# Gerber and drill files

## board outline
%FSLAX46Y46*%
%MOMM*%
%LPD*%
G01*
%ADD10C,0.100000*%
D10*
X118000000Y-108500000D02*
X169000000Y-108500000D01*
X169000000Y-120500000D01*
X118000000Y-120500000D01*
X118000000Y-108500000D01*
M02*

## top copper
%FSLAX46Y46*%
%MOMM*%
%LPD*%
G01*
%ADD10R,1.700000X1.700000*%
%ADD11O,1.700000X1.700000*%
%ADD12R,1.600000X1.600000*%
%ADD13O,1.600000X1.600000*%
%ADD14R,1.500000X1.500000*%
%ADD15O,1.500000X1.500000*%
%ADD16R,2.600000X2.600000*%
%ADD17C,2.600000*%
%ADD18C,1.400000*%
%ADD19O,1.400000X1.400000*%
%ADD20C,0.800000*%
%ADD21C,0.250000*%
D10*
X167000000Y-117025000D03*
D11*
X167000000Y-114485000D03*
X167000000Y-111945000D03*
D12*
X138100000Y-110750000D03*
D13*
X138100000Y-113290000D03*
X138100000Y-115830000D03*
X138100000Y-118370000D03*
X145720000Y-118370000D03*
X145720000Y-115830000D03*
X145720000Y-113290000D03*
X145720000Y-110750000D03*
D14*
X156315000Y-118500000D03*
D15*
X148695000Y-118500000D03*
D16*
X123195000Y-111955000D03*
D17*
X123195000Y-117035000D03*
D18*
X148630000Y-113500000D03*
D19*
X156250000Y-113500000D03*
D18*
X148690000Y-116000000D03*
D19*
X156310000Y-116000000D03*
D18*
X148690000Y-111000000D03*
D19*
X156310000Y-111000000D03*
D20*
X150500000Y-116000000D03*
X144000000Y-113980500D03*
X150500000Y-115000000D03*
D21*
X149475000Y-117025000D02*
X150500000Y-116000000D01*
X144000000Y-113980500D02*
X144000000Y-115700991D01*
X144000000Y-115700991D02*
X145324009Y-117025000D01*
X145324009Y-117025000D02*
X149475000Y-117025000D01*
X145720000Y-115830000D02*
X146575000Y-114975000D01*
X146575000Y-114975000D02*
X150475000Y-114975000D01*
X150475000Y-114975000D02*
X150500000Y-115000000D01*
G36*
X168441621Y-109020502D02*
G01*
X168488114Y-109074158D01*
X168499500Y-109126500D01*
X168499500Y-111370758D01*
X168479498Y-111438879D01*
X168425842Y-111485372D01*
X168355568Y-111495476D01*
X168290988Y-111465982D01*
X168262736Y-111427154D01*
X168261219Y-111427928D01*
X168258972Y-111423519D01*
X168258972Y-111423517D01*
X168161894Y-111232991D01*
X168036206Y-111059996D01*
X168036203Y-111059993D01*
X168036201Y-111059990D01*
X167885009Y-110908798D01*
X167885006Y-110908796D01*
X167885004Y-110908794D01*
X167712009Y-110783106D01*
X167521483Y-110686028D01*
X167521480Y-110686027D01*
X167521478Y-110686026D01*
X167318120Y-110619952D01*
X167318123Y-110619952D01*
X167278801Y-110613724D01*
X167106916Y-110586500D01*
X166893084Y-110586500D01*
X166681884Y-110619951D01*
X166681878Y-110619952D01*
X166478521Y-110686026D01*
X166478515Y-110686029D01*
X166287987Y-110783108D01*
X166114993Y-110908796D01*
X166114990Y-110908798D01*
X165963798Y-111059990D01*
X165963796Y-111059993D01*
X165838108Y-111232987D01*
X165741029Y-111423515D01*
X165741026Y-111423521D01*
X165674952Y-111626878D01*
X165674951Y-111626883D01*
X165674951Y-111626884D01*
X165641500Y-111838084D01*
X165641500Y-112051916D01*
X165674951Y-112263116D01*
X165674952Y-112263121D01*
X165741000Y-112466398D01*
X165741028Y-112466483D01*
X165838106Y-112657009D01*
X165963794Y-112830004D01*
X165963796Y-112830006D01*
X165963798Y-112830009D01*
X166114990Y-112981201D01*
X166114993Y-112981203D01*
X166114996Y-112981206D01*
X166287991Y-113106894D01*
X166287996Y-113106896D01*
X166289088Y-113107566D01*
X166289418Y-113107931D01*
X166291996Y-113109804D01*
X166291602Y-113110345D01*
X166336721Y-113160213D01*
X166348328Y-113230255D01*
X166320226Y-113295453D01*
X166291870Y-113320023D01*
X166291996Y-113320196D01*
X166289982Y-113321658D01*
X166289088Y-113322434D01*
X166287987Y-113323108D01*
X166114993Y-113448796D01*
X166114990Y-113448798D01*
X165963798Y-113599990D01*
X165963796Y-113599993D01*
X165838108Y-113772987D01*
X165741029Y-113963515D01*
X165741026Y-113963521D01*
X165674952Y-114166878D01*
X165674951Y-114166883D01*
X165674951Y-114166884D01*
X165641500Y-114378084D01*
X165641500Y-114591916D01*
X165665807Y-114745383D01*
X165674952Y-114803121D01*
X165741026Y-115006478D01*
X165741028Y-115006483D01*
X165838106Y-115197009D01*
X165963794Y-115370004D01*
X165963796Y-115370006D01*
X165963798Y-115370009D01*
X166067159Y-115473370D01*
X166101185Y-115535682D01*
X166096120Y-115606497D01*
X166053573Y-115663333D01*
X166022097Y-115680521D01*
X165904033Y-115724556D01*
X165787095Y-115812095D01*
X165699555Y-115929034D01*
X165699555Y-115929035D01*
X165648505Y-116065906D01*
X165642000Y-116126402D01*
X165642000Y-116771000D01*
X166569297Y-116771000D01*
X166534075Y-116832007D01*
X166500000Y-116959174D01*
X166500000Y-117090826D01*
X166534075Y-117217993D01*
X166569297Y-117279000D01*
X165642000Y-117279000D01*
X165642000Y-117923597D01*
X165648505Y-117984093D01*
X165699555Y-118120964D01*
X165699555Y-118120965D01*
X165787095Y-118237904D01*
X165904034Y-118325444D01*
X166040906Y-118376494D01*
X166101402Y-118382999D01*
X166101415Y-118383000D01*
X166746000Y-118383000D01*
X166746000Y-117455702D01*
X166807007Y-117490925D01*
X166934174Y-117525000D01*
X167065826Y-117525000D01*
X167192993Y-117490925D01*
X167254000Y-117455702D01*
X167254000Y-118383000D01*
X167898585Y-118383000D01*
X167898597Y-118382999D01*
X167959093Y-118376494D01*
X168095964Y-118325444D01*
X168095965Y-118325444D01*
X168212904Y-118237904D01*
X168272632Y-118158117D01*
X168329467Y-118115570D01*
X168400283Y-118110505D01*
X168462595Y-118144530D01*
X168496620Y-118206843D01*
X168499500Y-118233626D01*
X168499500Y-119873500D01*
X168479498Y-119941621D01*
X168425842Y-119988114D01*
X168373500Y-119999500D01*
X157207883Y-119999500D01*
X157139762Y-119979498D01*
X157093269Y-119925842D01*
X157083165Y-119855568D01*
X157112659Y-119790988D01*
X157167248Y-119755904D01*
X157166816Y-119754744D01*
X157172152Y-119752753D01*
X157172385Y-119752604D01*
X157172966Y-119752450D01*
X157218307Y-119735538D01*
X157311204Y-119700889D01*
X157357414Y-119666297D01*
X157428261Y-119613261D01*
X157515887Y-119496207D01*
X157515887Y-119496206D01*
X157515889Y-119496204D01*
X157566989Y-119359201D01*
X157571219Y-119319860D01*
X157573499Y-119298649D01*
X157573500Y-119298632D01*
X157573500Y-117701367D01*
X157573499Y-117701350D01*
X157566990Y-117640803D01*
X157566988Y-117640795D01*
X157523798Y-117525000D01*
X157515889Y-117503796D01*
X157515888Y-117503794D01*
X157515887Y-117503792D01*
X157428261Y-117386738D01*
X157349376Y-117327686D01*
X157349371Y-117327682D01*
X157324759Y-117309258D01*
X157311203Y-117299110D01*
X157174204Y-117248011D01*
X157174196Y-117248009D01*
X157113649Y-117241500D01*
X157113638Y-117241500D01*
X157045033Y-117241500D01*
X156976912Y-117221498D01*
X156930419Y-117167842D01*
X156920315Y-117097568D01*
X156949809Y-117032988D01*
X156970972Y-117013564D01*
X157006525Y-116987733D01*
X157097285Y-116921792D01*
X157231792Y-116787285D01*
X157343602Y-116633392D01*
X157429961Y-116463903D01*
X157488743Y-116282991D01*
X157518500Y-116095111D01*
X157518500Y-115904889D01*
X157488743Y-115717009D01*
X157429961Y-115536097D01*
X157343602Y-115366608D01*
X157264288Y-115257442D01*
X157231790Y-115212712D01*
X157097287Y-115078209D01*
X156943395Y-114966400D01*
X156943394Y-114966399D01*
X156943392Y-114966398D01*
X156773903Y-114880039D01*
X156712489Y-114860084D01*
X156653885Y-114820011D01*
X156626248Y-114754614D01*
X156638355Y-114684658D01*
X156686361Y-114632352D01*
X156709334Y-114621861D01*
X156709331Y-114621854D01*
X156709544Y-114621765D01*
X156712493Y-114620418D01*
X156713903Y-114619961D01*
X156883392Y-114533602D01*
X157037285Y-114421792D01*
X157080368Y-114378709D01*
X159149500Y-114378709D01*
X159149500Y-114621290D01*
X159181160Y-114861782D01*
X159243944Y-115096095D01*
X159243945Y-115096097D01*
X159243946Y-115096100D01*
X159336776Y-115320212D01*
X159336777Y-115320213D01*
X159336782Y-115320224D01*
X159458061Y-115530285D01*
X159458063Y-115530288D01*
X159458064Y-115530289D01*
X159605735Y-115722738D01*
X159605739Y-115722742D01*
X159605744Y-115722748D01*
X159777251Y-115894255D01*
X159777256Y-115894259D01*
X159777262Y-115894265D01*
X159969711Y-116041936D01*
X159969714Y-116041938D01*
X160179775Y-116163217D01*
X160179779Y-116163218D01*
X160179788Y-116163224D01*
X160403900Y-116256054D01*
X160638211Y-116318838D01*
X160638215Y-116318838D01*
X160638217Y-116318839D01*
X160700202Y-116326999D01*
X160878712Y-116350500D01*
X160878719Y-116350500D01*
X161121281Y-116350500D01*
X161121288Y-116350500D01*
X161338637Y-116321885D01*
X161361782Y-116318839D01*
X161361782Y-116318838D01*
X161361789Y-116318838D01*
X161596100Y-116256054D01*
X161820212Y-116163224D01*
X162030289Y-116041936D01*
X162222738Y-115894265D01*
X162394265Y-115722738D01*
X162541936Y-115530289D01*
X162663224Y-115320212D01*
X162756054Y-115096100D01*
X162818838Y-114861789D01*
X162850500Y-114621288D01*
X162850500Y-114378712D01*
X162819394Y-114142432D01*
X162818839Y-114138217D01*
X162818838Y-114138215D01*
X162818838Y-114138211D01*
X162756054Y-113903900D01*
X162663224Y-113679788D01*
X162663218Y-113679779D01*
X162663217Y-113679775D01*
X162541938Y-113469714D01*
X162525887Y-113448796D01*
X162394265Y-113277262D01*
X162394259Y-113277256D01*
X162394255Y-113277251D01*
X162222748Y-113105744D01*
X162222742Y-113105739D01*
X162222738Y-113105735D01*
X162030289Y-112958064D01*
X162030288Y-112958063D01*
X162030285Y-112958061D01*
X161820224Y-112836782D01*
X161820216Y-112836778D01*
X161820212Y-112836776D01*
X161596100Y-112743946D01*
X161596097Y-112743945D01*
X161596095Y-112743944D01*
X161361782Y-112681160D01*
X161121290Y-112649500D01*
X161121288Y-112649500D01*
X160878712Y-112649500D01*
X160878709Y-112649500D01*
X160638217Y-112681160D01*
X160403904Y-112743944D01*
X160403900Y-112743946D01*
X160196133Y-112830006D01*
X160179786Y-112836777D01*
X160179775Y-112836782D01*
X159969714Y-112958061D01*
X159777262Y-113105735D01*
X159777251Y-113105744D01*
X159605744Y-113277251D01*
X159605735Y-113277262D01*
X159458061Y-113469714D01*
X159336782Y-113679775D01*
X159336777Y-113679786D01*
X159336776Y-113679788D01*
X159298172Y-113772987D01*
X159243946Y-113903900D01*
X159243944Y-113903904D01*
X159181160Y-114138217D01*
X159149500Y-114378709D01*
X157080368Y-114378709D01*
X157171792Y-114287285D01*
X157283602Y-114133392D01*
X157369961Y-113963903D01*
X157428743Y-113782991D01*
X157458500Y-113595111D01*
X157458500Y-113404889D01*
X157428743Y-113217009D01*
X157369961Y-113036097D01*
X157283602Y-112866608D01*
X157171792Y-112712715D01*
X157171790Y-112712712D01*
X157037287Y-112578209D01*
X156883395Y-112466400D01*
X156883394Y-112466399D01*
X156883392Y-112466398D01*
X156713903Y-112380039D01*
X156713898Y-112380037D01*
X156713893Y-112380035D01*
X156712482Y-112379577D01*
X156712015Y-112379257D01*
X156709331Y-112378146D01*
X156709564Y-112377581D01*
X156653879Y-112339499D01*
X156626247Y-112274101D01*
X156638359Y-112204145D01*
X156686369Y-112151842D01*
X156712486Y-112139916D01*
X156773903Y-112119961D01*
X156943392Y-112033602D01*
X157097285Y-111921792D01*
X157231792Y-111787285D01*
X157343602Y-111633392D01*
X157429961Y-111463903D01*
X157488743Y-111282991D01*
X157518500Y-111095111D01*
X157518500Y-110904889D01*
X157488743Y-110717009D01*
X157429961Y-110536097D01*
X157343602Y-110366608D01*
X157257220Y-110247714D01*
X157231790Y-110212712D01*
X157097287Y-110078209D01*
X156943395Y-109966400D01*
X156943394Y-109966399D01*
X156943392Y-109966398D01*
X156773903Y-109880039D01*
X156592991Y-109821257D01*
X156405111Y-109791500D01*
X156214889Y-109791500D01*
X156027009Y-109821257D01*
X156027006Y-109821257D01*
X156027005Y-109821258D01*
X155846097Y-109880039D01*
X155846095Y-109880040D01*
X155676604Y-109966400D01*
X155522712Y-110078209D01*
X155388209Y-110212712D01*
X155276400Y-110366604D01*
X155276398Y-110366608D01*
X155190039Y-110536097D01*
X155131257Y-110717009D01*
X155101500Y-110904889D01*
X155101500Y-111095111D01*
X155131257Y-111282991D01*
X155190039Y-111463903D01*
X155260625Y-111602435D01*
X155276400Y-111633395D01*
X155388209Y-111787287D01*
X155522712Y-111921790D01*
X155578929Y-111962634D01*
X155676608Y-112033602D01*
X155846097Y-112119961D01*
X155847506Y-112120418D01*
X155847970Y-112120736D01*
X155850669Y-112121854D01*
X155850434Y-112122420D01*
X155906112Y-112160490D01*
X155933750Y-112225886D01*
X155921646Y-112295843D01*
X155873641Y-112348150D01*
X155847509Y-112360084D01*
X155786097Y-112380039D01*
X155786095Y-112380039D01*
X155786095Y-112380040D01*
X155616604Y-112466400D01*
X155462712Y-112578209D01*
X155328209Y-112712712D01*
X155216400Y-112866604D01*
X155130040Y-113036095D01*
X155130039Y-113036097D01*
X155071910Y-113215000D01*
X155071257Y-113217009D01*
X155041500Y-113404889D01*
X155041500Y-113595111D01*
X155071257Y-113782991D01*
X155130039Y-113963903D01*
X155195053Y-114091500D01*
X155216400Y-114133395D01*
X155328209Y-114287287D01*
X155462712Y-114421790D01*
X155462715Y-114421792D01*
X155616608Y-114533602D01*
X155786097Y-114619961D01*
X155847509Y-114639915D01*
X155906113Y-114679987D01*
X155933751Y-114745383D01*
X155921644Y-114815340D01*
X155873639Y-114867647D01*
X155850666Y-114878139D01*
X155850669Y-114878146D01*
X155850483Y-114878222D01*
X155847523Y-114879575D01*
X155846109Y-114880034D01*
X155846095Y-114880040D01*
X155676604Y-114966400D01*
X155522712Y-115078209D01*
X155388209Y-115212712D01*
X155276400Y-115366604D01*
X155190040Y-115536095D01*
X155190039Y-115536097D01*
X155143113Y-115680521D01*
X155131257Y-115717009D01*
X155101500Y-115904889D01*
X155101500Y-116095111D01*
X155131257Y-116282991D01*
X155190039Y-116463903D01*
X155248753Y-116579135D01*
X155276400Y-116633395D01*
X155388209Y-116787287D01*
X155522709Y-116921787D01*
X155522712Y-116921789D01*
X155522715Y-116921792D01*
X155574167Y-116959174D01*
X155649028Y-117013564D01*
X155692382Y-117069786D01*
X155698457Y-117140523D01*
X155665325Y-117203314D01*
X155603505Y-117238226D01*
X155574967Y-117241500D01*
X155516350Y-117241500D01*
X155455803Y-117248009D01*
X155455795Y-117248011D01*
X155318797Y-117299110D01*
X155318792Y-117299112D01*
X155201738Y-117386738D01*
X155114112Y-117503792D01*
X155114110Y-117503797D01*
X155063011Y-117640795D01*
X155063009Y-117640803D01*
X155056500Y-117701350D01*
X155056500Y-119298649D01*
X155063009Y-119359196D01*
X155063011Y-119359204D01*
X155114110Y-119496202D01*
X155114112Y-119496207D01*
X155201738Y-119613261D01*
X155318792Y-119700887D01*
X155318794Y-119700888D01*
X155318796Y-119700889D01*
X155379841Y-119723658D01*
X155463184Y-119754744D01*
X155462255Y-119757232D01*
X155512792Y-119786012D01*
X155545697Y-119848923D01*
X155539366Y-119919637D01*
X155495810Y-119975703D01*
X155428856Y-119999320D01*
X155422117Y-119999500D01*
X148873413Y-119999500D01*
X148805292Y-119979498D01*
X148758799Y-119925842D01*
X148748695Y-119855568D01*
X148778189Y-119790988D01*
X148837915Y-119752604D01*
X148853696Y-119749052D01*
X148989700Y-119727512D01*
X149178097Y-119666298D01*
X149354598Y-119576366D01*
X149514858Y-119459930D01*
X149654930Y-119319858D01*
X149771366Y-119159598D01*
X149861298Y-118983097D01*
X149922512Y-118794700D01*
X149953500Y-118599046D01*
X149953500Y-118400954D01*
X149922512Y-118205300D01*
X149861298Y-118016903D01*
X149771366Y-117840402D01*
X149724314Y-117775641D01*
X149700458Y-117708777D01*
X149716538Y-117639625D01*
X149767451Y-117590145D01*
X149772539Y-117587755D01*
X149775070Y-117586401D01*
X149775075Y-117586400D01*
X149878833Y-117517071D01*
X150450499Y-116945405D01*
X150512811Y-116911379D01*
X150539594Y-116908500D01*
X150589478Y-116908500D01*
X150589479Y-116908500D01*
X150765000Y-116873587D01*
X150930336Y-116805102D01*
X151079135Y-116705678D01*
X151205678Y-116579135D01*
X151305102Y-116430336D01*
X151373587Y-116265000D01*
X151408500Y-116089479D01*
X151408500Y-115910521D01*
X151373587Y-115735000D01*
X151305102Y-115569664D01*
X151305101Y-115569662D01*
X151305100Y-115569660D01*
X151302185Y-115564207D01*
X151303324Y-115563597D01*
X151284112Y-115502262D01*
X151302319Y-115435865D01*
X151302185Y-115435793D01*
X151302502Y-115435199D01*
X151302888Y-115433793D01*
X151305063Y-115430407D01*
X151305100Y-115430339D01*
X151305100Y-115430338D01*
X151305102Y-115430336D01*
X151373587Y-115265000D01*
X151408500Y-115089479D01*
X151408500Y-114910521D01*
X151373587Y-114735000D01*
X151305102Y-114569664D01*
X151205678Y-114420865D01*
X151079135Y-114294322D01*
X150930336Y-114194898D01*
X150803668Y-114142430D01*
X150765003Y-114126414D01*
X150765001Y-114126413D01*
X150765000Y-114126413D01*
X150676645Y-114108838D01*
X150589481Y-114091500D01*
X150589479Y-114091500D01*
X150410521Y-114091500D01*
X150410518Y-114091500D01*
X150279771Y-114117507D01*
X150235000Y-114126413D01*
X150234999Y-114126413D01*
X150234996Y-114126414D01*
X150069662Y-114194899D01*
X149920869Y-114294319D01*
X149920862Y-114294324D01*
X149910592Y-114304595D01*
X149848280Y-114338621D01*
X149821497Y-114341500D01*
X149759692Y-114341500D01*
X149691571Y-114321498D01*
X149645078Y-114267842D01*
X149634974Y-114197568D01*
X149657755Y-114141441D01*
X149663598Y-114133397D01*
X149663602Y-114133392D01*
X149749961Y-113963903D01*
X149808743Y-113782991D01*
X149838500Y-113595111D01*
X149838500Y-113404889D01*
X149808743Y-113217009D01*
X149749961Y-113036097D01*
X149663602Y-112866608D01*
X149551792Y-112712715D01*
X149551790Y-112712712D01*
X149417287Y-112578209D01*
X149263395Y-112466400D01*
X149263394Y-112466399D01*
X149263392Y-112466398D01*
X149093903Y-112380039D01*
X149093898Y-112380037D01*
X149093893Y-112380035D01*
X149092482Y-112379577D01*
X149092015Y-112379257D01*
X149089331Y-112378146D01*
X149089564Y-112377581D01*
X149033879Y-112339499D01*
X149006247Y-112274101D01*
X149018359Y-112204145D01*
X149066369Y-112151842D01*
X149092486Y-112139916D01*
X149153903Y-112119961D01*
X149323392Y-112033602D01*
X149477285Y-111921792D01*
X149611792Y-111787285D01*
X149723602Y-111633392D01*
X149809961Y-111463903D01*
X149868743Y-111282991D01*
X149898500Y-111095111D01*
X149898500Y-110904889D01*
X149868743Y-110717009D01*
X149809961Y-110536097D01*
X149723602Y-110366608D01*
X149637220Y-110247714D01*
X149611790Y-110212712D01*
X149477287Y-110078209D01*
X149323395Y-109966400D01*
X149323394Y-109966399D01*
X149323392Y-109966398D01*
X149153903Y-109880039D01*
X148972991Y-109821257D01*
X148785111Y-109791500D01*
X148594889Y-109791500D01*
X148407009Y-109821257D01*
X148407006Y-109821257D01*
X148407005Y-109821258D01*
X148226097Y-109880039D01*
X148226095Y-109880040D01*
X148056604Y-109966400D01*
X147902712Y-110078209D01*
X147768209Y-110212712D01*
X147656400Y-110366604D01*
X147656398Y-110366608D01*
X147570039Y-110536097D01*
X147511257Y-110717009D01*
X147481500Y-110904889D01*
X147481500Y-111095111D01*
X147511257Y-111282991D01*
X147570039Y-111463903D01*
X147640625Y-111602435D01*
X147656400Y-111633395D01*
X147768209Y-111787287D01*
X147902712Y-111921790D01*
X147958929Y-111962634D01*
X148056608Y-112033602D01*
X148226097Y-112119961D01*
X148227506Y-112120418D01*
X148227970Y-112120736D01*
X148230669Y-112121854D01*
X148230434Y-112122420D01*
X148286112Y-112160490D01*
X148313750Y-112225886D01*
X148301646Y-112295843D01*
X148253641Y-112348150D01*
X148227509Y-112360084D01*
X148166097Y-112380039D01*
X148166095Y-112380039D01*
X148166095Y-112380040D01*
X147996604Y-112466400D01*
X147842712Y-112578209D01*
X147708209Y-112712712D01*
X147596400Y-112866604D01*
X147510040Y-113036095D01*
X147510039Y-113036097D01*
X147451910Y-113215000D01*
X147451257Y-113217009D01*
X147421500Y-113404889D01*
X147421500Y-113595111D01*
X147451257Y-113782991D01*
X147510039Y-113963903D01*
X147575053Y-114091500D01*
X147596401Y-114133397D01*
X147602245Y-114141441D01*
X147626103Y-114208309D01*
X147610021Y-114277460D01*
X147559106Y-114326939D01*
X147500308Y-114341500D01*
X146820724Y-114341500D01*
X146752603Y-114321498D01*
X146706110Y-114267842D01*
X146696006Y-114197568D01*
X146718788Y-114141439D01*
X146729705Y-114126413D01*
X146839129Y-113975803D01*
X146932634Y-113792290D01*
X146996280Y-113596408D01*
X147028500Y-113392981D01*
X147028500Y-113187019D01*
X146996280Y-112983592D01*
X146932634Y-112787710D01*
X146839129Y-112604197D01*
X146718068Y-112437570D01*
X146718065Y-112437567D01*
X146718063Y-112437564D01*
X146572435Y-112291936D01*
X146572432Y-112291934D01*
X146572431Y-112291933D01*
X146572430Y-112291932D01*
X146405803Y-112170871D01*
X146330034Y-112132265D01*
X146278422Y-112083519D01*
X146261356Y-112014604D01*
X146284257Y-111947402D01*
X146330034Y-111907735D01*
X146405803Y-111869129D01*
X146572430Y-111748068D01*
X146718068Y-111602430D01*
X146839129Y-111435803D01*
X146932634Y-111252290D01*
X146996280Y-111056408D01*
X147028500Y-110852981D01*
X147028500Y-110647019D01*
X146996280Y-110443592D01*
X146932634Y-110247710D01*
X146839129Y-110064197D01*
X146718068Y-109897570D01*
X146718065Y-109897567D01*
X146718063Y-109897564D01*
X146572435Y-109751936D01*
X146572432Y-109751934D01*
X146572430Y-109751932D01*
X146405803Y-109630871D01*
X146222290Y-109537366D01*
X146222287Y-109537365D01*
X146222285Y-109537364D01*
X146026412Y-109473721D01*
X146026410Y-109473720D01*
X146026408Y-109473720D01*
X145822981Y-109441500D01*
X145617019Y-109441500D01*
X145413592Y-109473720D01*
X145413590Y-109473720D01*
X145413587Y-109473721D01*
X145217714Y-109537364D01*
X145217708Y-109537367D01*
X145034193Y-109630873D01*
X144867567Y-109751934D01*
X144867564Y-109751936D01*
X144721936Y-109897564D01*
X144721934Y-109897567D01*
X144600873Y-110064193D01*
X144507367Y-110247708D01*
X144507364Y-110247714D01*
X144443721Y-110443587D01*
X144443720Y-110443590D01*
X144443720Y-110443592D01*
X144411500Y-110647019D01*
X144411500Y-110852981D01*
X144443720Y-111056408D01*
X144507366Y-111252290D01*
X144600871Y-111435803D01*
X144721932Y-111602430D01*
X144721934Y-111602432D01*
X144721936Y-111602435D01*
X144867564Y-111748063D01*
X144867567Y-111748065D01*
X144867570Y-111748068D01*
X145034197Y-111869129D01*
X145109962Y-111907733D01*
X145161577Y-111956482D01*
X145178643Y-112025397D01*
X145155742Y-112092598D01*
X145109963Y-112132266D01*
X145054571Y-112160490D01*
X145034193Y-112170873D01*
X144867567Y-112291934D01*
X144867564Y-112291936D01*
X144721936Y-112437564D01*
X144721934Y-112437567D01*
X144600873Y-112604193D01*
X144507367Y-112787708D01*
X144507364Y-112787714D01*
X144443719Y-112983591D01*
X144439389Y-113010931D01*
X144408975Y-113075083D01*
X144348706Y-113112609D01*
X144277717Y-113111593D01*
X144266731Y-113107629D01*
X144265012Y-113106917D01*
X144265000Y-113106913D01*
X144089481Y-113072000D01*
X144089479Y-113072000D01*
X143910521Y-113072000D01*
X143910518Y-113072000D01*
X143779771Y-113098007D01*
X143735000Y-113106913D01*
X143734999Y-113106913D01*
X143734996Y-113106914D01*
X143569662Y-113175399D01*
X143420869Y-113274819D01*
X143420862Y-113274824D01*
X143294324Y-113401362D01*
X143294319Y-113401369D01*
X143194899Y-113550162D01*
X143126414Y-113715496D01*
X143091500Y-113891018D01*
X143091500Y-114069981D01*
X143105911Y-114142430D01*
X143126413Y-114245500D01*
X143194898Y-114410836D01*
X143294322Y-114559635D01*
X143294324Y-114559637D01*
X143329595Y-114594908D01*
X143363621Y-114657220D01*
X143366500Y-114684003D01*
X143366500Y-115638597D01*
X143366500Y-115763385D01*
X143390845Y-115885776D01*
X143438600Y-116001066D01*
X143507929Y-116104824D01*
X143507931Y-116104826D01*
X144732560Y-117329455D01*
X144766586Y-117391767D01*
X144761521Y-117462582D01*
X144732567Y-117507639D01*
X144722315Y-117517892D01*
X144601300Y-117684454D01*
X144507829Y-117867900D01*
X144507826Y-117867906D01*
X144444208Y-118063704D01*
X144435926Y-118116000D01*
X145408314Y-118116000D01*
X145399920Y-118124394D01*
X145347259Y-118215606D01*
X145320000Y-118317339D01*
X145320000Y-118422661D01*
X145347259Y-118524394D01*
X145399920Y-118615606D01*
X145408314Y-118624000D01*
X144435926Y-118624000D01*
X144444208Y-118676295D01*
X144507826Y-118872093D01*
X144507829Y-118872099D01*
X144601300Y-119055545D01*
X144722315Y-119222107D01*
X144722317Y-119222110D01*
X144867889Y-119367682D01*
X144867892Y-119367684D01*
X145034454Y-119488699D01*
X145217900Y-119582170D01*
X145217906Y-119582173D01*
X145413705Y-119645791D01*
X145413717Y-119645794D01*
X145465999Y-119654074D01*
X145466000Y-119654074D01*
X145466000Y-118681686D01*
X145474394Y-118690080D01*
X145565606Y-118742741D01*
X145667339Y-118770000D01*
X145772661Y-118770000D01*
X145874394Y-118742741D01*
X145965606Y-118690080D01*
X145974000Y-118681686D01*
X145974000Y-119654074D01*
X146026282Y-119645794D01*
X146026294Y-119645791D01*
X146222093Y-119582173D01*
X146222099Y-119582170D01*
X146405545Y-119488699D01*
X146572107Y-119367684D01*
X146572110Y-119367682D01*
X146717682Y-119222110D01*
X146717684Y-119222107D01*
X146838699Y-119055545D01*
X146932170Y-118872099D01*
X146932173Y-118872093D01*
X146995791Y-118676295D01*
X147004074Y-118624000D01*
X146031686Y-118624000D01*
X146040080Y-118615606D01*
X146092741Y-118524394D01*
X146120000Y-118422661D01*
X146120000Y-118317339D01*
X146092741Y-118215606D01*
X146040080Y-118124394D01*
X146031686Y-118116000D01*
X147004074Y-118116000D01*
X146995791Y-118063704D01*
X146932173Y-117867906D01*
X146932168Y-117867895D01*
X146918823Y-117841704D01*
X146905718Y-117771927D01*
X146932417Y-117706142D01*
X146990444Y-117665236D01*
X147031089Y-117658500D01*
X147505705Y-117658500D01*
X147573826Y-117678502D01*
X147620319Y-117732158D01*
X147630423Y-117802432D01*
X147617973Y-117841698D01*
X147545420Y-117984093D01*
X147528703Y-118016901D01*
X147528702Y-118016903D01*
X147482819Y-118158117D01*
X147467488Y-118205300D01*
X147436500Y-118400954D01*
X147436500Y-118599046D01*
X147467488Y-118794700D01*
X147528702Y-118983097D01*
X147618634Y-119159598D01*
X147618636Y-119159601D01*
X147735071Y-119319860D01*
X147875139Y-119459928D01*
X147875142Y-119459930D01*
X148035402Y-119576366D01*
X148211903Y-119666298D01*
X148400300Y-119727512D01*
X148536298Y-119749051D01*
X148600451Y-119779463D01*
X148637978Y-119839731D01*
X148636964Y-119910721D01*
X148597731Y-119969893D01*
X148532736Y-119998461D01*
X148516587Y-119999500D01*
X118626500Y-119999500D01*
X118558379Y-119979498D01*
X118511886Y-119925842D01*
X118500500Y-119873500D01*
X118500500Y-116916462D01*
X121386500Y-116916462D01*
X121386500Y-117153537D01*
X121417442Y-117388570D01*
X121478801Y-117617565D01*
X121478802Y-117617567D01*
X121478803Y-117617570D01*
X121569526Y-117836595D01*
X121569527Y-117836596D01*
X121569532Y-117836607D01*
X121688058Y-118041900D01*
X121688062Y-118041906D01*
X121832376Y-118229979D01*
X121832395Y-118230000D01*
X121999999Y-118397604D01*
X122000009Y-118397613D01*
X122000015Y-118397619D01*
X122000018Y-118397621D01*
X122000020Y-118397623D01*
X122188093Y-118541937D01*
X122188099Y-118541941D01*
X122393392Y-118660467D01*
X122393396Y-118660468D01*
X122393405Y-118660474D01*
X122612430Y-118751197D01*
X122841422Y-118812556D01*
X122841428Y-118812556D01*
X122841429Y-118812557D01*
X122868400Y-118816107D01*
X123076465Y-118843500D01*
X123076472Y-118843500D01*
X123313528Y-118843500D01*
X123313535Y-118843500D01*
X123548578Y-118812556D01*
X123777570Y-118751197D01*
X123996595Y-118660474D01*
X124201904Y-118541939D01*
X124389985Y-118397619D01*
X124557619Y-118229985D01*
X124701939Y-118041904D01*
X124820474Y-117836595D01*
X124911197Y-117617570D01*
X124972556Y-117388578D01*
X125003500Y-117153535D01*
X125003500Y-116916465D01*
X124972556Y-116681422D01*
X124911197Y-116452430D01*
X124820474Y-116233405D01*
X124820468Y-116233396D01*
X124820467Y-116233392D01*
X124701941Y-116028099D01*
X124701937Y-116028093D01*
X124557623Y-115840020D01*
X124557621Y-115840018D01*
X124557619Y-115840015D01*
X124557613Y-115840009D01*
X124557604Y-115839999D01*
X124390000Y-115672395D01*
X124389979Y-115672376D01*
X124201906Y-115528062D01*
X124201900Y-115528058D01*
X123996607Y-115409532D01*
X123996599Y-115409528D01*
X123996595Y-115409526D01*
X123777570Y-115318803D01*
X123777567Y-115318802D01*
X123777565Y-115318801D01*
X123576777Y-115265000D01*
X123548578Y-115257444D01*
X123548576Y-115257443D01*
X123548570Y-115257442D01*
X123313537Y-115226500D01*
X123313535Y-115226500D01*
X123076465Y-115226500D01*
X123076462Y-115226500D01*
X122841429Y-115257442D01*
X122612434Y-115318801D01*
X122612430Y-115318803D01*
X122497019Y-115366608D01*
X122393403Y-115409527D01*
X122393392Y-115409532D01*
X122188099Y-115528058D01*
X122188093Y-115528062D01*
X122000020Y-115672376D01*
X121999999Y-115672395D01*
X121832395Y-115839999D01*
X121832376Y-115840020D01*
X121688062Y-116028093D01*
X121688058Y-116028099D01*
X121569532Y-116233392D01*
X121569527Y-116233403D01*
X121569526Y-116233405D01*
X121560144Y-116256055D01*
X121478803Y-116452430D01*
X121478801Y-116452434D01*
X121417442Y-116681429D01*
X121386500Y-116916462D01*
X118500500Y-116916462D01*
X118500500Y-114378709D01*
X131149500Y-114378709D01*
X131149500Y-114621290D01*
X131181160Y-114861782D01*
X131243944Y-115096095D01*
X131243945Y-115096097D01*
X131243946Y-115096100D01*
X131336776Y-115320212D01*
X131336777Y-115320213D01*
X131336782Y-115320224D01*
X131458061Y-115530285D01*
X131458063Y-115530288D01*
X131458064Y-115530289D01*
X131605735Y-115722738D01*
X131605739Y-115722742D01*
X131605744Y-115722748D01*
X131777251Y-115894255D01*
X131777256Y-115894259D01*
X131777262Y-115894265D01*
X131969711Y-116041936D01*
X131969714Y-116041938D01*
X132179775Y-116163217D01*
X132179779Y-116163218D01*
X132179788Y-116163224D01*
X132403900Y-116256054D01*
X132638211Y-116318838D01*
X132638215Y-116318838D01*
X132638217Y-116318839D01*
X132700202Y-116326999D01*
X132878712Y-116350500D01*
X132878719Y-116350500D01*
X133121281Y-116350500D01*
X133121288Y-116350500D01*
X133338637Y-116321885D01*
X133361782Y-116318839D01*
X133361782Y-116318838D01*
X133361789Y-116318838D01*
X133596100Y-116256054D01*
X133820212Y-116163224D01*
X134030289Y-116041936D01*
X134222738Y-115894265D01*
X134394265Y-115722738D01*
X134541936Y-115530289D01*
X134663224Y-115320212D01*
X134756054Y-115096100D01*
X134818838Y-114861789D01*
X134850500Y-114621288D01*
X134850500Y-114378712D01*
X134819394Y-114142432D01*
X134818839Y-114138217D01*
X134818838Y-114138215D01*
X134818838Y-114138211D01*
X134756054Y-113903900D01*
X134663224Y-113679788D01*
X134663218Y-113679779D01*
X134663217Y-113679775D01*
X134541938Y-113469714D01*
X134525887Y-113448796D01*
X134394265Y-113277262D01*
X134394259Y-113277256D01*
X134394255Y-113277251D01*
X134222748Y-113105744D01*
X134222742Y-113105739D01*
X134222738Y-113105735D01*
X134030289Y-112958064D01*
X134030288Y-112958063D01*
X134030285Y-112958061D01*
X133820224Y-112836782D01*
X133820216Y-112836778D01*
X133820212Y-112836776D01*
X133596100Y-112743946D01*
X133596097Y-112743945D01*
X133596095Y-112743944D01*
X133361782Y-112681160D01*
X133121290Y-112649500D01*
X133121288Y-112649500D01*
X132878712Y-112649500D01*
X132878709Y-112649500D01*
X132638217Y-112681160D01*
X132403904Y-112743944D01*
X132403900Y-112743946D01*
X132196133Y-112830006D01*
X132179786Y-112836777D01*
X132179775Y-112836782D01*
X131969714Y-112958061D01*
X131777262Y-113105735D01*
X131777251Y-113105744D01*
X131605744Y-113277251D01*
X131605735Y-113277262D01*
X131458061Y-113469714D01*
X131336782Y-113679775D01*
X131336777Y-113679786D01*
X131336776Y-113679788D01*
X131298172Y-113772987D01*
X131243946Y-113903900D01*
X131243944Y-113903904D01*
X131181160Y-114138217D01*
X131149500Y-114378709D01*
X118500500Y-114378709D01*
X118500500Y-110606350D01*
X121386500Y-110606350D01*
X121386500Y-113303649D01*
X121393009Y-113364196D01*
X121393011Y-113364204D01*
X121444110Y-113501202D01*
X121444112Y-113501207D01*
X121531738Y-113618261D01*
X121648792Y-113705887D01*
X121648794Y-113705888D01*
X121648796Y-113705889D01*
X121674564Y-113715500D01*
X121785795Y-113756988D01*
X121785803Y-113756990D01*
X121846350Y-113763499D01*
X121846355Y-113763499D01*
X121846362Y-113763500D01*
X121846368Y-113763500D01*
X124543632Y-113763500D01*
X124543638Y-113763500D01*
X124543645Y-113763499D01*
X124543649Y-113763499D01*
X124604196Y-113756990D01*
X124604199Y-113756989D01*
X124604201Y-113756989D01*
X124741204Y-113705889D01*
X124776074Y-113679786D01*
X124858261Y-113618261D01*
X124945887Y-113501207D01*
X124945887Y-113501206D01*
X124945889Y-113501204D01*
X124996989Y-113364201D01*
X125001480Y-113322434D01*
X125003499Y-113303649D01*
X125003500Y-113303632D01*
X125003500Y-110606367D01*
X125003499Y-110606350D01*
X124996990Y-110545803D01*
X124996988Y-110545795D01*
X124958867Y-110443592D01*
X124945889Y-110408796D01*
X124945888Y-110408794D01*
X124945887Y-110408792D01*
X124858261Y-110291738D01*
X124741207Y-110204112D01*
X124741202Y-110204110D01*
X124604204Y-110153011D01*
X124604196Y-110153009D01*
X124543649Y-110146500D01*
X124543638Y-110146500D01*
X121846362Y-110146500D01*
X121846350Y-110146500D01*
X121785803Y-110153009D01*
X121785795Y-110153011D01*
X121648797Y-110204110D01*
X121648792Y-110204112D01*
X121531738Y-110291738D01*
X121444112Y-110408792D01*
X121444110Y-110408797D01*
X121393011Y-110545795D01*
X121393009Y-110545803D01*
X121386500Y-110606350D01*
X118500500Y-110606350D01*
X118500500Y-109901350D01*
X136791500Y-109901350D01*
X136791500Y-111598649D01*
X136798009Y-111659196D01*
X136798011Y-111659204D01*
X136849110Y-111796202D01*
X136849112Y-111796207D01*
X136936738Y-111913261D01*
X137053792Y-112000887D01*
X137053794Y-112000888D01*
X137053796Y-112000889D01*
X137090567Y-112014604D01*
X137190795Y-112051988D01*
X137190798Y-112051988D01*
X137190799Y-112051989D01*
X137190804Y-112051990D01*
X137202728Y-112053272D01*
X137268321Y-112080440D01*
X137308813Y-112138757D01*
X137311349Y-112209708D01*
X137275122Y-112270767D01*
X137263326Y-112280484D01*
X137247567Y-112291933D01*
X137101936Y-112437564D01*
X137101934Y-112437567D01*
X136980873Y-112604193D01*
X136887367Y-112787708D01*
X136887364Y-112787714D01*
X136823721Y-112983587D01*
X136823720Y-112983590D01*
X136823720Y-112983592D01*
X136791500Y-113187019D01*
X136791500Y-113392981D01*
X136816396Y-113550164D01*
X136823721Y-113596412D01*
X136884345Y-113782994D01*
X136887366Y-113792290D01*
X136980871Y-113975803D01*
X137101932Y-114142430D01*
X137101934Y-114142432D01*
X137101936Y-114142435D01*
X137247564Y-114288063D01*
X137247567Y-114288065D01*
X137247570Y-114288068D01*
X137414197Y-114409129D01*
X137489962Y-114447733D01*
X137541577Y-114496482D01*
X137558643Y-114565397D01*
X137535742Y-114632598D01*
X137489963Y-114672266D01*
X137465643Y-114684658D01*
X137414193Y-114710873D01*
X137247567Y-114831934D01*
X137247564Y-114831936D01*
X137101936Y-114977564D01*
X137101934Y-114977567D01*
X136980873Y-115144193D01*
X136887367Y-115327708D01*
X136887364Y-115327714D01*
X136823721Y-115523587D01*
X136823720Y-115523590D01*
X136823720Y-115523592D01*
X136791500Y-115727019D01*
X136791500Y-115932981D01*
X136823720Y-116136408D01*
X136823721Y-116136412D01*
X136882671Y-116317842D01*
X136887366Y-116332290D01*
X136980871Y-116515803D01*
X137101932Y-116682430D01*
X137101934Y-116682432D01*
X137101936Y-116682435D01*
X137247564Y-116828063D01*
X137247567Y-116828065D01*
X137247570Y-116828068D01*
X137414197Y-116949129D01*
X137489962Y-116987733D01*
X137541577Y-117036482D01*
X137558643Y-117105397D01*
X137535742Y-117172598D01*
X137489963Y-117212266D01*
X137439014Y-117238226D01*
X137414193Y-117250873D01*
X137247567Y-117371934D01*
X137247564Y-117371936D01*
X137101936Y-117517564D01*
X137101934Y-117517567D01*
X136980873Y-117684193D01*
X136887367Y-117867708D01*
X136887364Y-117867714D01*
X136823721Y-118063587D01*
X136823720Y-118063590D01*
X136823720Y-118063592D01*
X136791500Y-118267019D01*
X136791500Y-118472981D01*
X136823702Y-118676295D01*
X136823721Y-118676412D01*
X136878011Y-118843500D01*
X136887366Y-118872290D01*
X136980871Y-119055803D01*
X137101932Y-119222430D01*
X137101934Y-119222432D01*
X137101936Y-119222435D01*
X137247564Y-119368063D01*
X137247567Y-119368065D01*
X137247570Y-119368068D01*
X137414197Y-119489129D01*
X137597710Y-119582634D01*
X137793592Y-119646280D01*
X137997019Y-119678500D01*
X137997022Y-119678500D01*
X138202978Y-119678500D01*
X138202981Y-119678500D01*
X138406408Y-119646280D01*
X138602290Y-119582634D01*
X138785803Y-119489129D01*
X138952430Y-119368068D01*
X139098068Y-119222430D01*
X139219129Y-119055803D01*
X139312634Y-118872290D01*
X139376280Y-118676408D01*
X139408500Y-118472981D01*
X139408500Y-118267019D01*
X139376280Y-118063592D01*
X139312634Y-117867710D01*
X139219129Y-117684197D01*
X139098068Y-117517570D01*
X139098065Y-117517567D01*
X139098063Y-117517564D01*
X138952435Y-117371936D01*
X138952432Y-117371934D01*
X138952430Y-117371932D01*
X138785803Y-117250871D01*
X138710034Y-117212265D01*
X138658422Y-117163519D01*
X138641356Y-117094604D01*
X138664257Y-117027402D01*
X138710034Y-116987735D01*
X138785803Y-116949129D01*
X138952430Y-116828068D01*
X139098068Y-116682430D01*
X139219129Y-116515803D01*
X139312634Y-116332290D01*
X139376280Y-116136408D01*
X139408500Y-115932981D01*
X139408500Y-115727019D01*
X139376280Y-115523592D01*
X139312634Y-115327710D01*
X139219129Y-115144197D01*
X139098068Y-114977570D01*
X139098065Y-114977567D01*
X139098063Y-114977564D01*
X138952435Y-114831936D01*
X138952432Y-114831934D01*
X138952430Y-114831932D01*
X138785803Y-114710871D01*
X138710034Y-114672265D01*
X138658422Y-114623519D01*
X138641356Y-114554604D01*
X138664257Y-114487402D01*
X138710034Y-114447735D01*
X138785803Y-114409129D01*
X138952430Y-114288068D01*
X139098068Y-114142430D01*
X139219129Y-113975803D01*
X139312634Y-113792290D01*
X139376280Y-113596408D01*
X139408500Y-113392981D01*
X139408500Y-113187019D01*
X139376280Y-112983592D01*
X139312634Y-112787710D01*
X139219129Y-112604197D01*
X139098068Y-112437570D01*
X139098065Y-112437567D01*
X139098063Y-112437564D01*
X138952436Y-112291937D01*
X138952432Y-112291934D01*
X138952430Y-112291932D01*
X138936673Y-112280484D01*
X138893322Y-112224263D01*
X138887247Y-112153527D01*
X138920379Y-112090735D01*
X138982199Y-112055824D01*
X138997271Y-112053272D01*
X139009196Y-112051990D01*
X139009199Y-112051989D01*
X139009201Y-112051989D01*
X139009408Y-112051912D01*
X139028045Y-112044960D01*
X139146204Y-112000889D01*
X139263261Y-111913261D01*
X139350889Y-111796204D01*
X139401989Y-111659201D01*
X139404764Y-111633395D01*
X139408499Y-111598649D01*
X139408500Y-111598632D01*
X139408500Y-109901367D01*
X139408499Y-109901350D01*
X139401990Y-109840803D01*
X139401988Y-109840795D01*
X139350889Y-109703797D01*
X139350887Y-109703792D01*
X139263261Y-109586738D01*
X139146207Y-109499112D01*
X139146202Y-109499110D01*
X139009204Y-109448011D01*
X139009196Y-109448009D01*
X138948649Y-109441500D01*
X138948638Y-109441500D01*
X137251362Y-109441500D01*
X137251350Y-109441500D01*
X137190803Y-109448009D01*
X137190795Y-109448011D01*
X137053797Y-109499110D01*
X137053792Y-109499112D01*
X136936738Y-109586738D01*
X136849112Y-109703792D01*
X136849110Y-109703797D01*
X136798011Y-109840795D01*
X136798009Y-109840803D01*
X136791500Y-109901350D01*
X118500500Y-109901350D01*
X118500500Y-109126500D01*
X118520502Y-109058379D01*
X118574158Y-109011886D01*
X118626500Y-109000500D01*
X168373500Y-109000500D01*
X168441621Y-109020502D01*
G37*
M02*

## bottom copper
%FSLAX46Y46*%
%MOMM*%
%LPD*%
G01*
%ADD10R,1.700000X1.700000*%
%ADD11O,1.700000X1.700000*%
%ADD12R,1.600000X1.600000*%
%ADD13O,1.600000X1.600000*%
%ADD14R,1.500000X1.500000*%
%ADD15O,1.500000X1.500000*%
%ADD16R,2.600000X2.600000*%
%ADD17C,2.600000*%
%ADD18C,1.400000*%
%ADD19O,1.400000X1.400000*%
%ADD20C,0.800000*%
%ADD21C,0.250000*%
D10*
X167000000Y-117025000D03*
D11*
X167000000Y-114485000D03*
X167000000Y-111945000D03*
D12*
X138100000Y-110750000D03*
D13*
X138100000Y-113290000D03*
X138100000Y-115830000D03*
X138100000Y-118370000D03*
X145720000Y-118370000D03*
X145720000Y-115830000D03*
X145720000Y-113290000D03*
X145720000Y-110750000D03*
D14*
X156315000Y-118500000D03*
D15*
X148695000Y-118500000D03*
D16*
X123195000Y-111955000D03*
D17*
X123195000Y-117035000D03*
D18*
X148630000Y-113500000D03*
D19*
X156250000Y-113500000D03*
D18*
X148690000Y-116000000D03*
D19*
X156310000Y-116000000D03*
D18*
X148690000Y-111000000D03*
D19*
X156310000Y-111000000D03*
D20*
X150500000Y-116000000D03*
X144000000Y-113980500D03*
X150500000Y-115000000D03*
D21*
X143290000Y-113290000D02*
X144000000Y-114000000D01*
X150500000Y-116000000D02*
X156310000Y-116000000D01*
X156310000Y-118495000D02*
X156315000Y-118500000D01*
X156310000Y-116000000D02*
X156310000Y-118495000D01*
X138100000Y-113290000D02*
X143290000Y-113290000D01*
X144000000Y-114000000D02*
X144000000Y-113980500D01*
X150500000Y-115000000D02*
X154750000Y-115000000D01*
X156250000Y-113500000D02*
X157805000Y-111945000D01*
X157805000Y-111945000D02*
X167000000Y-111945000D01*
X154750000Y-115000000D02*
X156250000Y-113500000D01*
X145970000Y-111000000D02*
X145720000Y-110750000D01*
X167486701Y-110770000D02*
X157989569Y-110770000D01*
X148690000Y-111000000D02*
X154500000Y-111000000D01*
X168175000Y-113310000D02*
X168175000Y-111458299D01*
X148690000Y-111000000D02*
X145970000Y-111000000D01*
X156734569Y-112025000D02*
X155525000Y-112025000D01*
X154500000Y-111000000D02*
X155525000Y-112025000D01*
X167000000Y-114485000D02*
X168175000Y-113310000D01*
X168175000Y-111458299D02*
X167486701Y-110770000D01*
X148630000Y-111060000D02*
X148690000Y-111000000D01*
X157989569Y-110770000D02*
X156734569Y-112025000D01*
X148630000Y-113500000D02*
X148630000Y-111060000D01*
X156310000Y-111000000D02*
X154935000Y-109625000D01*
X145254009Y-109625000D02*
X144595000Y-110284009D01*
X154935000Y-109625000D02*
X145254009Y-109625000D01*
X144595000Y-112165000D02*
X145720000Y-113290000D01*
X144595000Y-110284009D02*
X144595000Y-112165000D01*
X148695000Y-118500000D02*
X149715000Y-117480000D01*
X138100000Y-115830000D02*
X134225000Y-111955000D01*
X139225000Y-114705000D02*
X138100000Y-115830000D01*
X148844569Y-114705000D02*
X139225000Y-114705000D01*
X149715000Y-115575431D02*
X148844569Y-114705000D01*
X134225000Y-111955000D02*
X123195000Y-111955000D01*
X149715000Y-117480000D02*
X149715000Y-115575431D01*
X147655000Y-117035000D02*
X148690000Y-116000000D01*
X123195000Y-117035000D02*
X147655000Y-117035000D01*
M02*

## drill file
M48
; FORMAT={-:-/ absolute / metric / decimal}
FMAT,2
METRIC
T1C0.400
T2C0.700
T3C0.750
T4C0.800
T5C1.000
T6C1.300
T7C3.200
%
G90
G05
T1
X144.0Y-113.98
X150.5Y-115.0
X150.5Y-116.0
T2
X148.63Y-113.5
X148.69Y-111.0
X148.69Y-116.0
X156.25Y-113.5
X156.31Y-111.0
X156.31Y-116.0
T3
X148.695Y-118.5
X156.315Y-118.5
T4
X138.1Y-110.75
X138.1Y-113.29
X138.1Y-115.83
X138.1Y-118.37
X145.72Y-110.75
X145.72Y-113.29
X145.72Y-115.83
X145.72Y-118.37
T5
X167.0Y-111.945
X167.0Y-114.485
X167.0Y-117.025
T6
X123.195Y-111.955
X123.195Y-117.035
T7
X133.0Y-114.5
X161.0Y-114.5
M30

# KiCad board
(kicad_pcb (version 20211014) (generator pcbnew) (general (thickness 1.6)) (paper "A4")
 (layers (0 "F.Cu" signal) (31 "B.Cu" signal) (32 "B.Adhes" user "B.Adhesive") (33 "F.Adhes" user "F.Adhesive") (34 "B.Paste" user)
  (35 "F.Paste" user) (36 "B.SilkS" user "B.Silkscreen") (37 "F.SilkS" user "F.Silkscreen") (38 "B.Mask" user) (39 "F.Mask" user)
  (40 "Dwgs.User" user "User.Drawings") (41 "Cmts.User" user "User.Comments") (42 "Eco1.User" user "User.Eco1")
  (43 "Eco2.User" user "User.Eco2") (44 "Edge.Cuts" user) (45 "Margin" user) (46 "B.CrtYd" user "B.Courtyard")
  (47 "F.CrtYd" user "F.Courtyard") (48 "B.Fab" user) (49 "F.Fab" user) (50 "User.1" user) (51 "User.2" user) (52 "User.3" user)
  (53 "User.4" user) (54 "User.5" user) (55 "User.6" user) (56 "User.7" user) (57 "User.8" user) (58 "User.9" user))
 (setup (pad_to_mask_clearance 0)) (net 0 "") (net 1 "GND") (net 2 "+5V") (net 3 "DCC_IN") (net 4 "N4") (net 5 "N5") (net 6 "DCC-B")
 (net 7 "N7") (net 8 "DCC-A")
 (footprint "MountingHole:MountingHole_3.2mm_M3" (layer "F.Cu") (at 133 114.5)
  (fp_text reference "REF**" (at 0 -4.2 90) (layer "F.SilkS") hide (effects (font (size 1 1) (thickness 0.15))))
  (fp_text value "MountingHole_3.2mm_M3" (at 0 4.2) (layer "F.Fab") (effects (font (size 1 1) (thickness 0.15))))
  (pad "" np_thru_hole circle (at 0 0) (size 3.2 3.2) (drill 3.2) (layers *.Cu *.Mask)))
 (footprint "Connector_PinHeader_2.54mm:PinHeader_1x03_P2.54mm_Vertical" (layer "F.Cu") (at 167 117.025 180)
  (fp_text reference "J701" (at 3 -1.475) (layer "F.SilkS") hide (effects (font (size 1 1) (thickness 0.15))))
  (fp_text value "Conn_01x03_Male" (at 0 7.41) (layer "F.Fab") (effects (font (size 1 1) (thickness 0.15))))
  (pad "1" thru_hole rect (at 0 0 180) (size 1.7 1.7) (drill 1) (layers *.Cu *.Mask) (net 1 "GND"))
  (pad "2" thru_hole oval (at 0 2.54 180) (size 1.7 1.7) (drill 1) (layers *.Cu *.Mask) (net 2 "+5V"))
  (pad "3" thru_hole oval (at 0 5.08 180) (size 1.7 1.7) (drill 1) (layers *.Cu *.Mask) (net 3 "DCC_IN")))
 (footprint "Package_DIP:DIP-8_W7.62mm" (layer "F.Cu") (at 138.1 110.75)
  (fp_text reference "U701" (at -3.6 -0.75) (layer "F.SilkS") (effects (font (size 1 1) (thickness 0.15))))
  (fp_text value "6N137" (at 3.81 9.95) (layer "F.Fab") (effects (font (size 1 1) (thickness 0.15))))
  (pad "1" thru_hole rect (at 0 0) (size 1.6 1.6) (drill 0.8) (layers *.Cu *.Mask) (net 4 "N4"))
  (pad "2" thru_hole oval (at 0 2.54) (size 1.6 1.6) (drill 0.8) (layers *.Cu *.Mask) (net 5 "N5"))
  (pad "3" thru_hole oval (at 0 5.08) (size 1.6 1.6) (drill 0.8) (layers *.Cu *.Mask) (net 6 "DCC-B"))
  (pad "4" thru_hole oval (at 0 7.62) (size 1.6 1.6) (drill 0.8) (layers *.Cu *.Mask))
  (pad "5" thru_hole oval (at 7.62 7.62) (size 1.6 1.6) (drill 0.8) (layers *.Cu *.Mask) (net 1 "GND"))
  (pad "6" thru_hole oval (at 7.62 5.08) (size 1.6 1.6) (drill 0.8) (layers *.Cu *.Mask) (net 3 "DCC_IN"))
  (pad "7" thru_hole oval (at 7.62 2.54) (size 1.6 1.6) (drill 0.8) (layers *.Cu *.Mask) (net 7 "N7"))
  (pad "8" thru_hole oval (at 7.62 0) (size 1.6 1.6) (drill 0.8) (layers *.Cu *.Mask) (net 2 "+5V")))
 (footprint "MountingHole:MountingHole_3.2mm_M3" (layer "F.Cu") (at 161 114.5)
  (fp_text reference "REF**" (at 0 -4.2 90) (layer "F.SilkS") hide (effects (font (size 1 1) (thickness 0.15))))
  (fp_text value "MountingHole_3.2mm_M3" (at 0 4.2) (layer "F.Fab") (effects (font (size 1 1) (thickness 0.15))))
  (pad "" np_thru_hole circle (at 0 0) (size 3.2 3.2) (drill 3.2) (layers F&B.Cu *.Mask)))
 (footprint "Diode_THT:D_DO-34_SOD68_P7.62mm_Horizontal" (layer "F.Cu") (at 156.315 118.5 180)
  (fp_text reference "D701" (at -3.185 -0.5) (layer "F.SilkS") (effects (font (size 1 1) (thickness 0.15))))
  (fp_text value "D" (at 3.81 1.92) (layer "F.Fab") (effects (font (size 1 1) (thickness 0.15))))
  (pad "1" thru_hole rect (at 0 0 180) (size 1.5 1.5) (drill 0.75) (layers *.Cu *.Mask) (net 5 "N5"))
  (pad "2" thru_hole oval (at 7.62 0 180) (size 1.5 1.5) (drill 0.75) (layers *.Cu *.Mask) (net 6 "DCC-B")))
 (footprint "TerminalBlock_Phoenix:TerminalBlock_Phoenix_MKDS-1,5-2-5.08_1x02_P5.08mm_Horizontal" (layer "F.Cu") (at 123.195 111.955 -90)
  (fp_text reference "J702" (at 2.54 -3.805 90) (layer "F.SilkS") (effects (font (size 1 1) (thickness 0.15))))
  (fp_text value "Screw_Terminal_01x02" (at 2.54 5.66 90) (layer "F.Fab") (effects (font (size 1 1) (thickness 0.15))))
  (pad "1" thru_hole rect (at 0 0 270) (size 2.6 2.6) (drill 1.3) (layers *.Cu *.Mask) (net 6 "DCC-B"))
  (pad "2" thru_hole circle (at 5.08 0 270) (size 2.6 2.6) (drill 1.3) (layers *.Cu *.Mask) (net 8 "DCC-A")))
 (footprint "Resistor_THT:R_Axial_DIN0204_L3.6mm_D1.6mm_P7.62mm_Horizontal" (layer "F.Cu") (at 148.63 113.5)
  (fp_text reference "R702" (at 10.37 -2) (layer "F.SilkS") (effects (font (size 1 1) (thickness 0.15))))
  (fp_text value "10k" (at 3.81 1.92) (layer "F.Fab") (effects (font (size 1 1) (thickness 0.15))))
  (pad "1" thru_hole circle (at 0 0) (size 1.4 1.4) (drill 0.7) (layers *.Cu *.Mask) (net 2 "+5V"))
  (pad "2" thru_hole oval (at 7.62 0) (size 1.4 1.4) (drill 0.7) (layers *.Cu *.Mask) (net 3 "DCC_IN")))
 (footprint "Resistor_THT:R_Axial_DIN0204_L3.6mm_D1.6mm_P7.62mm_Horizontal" (layer "F.Cu") (at 148.69 116)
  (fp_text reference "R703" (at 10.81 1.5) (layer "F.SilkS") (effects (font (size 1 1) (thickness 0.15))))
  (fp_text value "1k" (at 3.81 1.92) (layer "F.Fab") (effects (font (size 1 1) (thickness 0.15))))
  (pad "1" thru_hole circle (at 0 0) (size 1.4 1.4) (drill 0.7) (layers *.Cu *.Mask) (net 8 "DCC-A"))
  (pad "2" thru_hole oval (at 7.62 0) (size 1.4 1.4) (drill 0.7) (layers *.Cu *.Mask) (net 5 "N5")))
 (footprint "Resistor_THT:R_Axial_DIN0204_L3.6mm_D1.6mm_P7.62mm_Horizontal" (layer "F.Cu") (at 148.69 111)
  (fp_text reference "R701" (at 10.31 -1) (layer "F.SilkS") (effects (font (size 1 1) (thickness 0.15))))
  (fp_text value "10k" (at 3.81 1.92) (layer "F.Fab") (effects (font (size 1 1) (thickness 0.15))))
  (pad "1" thru_hole circle (at 0 0) (size 1.4 1.4) (drill 0.7) (layers *.Cu *.Mask) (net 2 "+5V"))
  (pad "2" thru_hole oval (at 7.62 0) (size 1.4 1.4) (drill 0.7) (layers *.Cu *.Mask) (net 7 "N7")))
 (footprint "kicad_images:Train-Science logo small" (layer "B.Cu") (at 125 114.5 90)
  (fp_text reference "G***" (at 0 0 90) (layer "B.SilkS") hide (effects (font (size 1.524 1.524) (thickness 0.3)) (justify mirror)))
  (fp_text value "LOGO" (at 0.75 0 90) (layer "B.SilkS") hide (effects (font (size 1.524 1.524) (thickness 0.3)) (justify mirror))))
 (gr_rect (start 169 120.5) (end 118 108.5) (layer "Edge.Cuts") (width 0.1) (fill none))
 (segment (start 149.475 117.025) (end 150.5 116) (width 0.25) (layer "F.Cu") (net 5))
 (segment (start 144 113.9805) (end 144 115.700991) (width 0.25) (layer "F.Cu") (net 5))
 (segment (start 144 115.700991) (end 145.324009 117.025) (width 0.25) (layer "F.Cu") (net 5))
 (segment (start 145.324009 117.025) (end 149.475 117.025) (width 0.25) (layer "F.Cu") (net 5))
 (via (at 150.5 116) (size 0.8) (drill 0.4) (layers "F.Cu" "B.Cu") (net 5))
 (via (at 144 113.9805) (size 0.8) (drill 0.4) (layers "F.Cu" "B.Cu") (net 5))
 (segment (start 143.29 113.29) (end 144 114) (width 0.25) (layer "B.Cu") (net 5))
 (segment (start 150.5 116) (end 156.31 116) (width 0.25) (layer "B.Cu") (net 5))
 (segment (start 156.31 118.495) (end 156.315 118.5) (width 0.25) (layer "B.Cu") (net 5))
 (segment (start 156.31 116) (end 156.31 118.495) (width 0.25) (layer "B.Cu") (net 5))
 (segment (start 138.1 113.29) (end 143.29 113.29) (width 0.25) (layer "B.Cu") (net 5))
 (segment (start 144 114) (end 144 113.9805) (width 0.25) (layer "B.Cu") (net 5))
 (segment (start 145.72 115.83) (end 146.575 114.975) (width 0.25) (layer "F.Cu") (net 3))
 (segment (start 146.575 114.975) (end 150.475 114.975) (width 0.25) (layer "F.Cu") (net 3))
 (segment (start 150.475 114.975) (end 150.5 115) (width 0.25) (layer "F.Cu") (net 3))
 (via (at 150.5 115) (size 0.8) (drill 0.4) (layers "F.Cu" "B.Cu") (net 3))
 (segment (start 150.5 115) (end 154.75 115) (width 0.25) (layer "B.Cu") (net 3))
 (segment (start 156.25 113.5) (end 157.805 111.945) (width 0.25) (layer "B.Cu") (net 3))
 (segment (start 157.805 111.945) (end 167 111.945) (width 0.25) (layer "B.Cu") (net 3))
 (segment (start 154.75 115) (end 156.25 113.5) (width 0.25) (layer "B.Cu") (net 3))
 (segment (start 145.97 111) (end 145.72 110.75) (width 0.25) (layer "B.Cu") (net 2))
 (segment (start 167.486701 110.77) (end 157.989569 110.77) (width 0.25) (layer "B.Cu") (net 2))
 (segment (start 148.69 111) (end 154.5 111) (width 0.25) (layer "B.Cu") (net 2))
 (segment (start 168.175 113.31) (end 168.175 111.458299) (width 0.25) (layer "B.Cu") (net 2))
 (segment (start 148.69 111) (end 145.97 111) (width 0.25) (layer "B.Cu") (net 2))
 (segment (start 156.734569 112.025) (end 155.525 112.025) (width 0.25) (layer "B.Cu") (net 2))
 (segment (start 154.5 111) (end 155.525 112.025) (width 0.25) (layer "B.Cu") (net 2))
 (segment (start 167 114.485) (end 168.175 113.31) (width 0.25) (layer "B.Cu") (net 2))
 (segment (start 168.175 111.458299) (end 167.486701 110.77) (width 0.25) (layer "B.Cu") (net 2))
 (segment (start 148.63 111.06) (end 148.69 111) (width 0.25) (layer "B.Cu") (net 2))
 (segment (start 157.989569 110.77) (end 156.734569 112.025) (width 0.25) (layer "B.Cu") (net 2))
 (segment (start 148.63 113.5) (end 148.63 111.06) (width 0.25) (layer "B.Cu") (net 2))
 (segment (start 156.31 111) (end 154.935 109.625) (width 0.25) (layer "B.Cu") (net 7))
 (segment (start 145.254009 109.625) (end 144.595 110.284009) (width 0.25) (layer "B.Cu") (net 7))
 (segment (start 154.935 109.625) (end 145.254009 109.625) (width 0.25) (layer "B.Cu") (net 7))
 (segment (start 144.595 112.165) (end 145.72 113.29) (width 0.25) (layer "B.Cu") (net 7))
 (segment (start 144.595 110.284009) (end 144.595 112.165) (width 0.25) (layer "B.Cu") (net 7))
 (segment (start 148.695 118.5) (end 149.715 117.48) (width 0.25) (layer "B.Cu") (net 6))
 (segment (start 138.1 115.83) (end 134.225 111.955) (width 0.25) (layer "B.Cu") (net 6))
 (segment (start 139.225 114.705) (end 138.1 115.83) (width 0.25) (layer "B.Cu") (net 6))
 (segment (start 148.844569 114.705) (end 139.225 114.705) (width 0.25) (layer "B.Cu") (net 6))
 (segment (start 149.715 115.575431) (end 148.844569 114.705) (width 0.25) (layer "B.Cu") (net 6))
 (segment (start 134.225 111.955) (end 123.195 111.955) (width 0.25) (layer "B.Cu") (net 6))
 (segment (start 149.715 117.48) (end 149.715 115.575431) (width 0.25) (layer "B.Cu") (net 6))
 (segment (start 147.655 117.035) (end 148.69 116) (width 0.25) (layer "B.Cu") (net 8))
 (segment (start 123.195 117.035) (end 147.655 117.035) (width 0.25) (layer "B.Cu") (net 8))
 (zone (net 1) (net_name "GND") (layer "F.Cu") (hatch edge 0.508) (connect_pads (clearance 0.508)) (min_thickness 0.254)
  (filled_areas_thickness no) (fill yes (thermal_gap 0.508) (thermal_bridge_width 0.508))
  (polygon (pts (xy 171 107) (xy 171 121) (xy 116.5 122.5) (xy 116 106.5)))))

